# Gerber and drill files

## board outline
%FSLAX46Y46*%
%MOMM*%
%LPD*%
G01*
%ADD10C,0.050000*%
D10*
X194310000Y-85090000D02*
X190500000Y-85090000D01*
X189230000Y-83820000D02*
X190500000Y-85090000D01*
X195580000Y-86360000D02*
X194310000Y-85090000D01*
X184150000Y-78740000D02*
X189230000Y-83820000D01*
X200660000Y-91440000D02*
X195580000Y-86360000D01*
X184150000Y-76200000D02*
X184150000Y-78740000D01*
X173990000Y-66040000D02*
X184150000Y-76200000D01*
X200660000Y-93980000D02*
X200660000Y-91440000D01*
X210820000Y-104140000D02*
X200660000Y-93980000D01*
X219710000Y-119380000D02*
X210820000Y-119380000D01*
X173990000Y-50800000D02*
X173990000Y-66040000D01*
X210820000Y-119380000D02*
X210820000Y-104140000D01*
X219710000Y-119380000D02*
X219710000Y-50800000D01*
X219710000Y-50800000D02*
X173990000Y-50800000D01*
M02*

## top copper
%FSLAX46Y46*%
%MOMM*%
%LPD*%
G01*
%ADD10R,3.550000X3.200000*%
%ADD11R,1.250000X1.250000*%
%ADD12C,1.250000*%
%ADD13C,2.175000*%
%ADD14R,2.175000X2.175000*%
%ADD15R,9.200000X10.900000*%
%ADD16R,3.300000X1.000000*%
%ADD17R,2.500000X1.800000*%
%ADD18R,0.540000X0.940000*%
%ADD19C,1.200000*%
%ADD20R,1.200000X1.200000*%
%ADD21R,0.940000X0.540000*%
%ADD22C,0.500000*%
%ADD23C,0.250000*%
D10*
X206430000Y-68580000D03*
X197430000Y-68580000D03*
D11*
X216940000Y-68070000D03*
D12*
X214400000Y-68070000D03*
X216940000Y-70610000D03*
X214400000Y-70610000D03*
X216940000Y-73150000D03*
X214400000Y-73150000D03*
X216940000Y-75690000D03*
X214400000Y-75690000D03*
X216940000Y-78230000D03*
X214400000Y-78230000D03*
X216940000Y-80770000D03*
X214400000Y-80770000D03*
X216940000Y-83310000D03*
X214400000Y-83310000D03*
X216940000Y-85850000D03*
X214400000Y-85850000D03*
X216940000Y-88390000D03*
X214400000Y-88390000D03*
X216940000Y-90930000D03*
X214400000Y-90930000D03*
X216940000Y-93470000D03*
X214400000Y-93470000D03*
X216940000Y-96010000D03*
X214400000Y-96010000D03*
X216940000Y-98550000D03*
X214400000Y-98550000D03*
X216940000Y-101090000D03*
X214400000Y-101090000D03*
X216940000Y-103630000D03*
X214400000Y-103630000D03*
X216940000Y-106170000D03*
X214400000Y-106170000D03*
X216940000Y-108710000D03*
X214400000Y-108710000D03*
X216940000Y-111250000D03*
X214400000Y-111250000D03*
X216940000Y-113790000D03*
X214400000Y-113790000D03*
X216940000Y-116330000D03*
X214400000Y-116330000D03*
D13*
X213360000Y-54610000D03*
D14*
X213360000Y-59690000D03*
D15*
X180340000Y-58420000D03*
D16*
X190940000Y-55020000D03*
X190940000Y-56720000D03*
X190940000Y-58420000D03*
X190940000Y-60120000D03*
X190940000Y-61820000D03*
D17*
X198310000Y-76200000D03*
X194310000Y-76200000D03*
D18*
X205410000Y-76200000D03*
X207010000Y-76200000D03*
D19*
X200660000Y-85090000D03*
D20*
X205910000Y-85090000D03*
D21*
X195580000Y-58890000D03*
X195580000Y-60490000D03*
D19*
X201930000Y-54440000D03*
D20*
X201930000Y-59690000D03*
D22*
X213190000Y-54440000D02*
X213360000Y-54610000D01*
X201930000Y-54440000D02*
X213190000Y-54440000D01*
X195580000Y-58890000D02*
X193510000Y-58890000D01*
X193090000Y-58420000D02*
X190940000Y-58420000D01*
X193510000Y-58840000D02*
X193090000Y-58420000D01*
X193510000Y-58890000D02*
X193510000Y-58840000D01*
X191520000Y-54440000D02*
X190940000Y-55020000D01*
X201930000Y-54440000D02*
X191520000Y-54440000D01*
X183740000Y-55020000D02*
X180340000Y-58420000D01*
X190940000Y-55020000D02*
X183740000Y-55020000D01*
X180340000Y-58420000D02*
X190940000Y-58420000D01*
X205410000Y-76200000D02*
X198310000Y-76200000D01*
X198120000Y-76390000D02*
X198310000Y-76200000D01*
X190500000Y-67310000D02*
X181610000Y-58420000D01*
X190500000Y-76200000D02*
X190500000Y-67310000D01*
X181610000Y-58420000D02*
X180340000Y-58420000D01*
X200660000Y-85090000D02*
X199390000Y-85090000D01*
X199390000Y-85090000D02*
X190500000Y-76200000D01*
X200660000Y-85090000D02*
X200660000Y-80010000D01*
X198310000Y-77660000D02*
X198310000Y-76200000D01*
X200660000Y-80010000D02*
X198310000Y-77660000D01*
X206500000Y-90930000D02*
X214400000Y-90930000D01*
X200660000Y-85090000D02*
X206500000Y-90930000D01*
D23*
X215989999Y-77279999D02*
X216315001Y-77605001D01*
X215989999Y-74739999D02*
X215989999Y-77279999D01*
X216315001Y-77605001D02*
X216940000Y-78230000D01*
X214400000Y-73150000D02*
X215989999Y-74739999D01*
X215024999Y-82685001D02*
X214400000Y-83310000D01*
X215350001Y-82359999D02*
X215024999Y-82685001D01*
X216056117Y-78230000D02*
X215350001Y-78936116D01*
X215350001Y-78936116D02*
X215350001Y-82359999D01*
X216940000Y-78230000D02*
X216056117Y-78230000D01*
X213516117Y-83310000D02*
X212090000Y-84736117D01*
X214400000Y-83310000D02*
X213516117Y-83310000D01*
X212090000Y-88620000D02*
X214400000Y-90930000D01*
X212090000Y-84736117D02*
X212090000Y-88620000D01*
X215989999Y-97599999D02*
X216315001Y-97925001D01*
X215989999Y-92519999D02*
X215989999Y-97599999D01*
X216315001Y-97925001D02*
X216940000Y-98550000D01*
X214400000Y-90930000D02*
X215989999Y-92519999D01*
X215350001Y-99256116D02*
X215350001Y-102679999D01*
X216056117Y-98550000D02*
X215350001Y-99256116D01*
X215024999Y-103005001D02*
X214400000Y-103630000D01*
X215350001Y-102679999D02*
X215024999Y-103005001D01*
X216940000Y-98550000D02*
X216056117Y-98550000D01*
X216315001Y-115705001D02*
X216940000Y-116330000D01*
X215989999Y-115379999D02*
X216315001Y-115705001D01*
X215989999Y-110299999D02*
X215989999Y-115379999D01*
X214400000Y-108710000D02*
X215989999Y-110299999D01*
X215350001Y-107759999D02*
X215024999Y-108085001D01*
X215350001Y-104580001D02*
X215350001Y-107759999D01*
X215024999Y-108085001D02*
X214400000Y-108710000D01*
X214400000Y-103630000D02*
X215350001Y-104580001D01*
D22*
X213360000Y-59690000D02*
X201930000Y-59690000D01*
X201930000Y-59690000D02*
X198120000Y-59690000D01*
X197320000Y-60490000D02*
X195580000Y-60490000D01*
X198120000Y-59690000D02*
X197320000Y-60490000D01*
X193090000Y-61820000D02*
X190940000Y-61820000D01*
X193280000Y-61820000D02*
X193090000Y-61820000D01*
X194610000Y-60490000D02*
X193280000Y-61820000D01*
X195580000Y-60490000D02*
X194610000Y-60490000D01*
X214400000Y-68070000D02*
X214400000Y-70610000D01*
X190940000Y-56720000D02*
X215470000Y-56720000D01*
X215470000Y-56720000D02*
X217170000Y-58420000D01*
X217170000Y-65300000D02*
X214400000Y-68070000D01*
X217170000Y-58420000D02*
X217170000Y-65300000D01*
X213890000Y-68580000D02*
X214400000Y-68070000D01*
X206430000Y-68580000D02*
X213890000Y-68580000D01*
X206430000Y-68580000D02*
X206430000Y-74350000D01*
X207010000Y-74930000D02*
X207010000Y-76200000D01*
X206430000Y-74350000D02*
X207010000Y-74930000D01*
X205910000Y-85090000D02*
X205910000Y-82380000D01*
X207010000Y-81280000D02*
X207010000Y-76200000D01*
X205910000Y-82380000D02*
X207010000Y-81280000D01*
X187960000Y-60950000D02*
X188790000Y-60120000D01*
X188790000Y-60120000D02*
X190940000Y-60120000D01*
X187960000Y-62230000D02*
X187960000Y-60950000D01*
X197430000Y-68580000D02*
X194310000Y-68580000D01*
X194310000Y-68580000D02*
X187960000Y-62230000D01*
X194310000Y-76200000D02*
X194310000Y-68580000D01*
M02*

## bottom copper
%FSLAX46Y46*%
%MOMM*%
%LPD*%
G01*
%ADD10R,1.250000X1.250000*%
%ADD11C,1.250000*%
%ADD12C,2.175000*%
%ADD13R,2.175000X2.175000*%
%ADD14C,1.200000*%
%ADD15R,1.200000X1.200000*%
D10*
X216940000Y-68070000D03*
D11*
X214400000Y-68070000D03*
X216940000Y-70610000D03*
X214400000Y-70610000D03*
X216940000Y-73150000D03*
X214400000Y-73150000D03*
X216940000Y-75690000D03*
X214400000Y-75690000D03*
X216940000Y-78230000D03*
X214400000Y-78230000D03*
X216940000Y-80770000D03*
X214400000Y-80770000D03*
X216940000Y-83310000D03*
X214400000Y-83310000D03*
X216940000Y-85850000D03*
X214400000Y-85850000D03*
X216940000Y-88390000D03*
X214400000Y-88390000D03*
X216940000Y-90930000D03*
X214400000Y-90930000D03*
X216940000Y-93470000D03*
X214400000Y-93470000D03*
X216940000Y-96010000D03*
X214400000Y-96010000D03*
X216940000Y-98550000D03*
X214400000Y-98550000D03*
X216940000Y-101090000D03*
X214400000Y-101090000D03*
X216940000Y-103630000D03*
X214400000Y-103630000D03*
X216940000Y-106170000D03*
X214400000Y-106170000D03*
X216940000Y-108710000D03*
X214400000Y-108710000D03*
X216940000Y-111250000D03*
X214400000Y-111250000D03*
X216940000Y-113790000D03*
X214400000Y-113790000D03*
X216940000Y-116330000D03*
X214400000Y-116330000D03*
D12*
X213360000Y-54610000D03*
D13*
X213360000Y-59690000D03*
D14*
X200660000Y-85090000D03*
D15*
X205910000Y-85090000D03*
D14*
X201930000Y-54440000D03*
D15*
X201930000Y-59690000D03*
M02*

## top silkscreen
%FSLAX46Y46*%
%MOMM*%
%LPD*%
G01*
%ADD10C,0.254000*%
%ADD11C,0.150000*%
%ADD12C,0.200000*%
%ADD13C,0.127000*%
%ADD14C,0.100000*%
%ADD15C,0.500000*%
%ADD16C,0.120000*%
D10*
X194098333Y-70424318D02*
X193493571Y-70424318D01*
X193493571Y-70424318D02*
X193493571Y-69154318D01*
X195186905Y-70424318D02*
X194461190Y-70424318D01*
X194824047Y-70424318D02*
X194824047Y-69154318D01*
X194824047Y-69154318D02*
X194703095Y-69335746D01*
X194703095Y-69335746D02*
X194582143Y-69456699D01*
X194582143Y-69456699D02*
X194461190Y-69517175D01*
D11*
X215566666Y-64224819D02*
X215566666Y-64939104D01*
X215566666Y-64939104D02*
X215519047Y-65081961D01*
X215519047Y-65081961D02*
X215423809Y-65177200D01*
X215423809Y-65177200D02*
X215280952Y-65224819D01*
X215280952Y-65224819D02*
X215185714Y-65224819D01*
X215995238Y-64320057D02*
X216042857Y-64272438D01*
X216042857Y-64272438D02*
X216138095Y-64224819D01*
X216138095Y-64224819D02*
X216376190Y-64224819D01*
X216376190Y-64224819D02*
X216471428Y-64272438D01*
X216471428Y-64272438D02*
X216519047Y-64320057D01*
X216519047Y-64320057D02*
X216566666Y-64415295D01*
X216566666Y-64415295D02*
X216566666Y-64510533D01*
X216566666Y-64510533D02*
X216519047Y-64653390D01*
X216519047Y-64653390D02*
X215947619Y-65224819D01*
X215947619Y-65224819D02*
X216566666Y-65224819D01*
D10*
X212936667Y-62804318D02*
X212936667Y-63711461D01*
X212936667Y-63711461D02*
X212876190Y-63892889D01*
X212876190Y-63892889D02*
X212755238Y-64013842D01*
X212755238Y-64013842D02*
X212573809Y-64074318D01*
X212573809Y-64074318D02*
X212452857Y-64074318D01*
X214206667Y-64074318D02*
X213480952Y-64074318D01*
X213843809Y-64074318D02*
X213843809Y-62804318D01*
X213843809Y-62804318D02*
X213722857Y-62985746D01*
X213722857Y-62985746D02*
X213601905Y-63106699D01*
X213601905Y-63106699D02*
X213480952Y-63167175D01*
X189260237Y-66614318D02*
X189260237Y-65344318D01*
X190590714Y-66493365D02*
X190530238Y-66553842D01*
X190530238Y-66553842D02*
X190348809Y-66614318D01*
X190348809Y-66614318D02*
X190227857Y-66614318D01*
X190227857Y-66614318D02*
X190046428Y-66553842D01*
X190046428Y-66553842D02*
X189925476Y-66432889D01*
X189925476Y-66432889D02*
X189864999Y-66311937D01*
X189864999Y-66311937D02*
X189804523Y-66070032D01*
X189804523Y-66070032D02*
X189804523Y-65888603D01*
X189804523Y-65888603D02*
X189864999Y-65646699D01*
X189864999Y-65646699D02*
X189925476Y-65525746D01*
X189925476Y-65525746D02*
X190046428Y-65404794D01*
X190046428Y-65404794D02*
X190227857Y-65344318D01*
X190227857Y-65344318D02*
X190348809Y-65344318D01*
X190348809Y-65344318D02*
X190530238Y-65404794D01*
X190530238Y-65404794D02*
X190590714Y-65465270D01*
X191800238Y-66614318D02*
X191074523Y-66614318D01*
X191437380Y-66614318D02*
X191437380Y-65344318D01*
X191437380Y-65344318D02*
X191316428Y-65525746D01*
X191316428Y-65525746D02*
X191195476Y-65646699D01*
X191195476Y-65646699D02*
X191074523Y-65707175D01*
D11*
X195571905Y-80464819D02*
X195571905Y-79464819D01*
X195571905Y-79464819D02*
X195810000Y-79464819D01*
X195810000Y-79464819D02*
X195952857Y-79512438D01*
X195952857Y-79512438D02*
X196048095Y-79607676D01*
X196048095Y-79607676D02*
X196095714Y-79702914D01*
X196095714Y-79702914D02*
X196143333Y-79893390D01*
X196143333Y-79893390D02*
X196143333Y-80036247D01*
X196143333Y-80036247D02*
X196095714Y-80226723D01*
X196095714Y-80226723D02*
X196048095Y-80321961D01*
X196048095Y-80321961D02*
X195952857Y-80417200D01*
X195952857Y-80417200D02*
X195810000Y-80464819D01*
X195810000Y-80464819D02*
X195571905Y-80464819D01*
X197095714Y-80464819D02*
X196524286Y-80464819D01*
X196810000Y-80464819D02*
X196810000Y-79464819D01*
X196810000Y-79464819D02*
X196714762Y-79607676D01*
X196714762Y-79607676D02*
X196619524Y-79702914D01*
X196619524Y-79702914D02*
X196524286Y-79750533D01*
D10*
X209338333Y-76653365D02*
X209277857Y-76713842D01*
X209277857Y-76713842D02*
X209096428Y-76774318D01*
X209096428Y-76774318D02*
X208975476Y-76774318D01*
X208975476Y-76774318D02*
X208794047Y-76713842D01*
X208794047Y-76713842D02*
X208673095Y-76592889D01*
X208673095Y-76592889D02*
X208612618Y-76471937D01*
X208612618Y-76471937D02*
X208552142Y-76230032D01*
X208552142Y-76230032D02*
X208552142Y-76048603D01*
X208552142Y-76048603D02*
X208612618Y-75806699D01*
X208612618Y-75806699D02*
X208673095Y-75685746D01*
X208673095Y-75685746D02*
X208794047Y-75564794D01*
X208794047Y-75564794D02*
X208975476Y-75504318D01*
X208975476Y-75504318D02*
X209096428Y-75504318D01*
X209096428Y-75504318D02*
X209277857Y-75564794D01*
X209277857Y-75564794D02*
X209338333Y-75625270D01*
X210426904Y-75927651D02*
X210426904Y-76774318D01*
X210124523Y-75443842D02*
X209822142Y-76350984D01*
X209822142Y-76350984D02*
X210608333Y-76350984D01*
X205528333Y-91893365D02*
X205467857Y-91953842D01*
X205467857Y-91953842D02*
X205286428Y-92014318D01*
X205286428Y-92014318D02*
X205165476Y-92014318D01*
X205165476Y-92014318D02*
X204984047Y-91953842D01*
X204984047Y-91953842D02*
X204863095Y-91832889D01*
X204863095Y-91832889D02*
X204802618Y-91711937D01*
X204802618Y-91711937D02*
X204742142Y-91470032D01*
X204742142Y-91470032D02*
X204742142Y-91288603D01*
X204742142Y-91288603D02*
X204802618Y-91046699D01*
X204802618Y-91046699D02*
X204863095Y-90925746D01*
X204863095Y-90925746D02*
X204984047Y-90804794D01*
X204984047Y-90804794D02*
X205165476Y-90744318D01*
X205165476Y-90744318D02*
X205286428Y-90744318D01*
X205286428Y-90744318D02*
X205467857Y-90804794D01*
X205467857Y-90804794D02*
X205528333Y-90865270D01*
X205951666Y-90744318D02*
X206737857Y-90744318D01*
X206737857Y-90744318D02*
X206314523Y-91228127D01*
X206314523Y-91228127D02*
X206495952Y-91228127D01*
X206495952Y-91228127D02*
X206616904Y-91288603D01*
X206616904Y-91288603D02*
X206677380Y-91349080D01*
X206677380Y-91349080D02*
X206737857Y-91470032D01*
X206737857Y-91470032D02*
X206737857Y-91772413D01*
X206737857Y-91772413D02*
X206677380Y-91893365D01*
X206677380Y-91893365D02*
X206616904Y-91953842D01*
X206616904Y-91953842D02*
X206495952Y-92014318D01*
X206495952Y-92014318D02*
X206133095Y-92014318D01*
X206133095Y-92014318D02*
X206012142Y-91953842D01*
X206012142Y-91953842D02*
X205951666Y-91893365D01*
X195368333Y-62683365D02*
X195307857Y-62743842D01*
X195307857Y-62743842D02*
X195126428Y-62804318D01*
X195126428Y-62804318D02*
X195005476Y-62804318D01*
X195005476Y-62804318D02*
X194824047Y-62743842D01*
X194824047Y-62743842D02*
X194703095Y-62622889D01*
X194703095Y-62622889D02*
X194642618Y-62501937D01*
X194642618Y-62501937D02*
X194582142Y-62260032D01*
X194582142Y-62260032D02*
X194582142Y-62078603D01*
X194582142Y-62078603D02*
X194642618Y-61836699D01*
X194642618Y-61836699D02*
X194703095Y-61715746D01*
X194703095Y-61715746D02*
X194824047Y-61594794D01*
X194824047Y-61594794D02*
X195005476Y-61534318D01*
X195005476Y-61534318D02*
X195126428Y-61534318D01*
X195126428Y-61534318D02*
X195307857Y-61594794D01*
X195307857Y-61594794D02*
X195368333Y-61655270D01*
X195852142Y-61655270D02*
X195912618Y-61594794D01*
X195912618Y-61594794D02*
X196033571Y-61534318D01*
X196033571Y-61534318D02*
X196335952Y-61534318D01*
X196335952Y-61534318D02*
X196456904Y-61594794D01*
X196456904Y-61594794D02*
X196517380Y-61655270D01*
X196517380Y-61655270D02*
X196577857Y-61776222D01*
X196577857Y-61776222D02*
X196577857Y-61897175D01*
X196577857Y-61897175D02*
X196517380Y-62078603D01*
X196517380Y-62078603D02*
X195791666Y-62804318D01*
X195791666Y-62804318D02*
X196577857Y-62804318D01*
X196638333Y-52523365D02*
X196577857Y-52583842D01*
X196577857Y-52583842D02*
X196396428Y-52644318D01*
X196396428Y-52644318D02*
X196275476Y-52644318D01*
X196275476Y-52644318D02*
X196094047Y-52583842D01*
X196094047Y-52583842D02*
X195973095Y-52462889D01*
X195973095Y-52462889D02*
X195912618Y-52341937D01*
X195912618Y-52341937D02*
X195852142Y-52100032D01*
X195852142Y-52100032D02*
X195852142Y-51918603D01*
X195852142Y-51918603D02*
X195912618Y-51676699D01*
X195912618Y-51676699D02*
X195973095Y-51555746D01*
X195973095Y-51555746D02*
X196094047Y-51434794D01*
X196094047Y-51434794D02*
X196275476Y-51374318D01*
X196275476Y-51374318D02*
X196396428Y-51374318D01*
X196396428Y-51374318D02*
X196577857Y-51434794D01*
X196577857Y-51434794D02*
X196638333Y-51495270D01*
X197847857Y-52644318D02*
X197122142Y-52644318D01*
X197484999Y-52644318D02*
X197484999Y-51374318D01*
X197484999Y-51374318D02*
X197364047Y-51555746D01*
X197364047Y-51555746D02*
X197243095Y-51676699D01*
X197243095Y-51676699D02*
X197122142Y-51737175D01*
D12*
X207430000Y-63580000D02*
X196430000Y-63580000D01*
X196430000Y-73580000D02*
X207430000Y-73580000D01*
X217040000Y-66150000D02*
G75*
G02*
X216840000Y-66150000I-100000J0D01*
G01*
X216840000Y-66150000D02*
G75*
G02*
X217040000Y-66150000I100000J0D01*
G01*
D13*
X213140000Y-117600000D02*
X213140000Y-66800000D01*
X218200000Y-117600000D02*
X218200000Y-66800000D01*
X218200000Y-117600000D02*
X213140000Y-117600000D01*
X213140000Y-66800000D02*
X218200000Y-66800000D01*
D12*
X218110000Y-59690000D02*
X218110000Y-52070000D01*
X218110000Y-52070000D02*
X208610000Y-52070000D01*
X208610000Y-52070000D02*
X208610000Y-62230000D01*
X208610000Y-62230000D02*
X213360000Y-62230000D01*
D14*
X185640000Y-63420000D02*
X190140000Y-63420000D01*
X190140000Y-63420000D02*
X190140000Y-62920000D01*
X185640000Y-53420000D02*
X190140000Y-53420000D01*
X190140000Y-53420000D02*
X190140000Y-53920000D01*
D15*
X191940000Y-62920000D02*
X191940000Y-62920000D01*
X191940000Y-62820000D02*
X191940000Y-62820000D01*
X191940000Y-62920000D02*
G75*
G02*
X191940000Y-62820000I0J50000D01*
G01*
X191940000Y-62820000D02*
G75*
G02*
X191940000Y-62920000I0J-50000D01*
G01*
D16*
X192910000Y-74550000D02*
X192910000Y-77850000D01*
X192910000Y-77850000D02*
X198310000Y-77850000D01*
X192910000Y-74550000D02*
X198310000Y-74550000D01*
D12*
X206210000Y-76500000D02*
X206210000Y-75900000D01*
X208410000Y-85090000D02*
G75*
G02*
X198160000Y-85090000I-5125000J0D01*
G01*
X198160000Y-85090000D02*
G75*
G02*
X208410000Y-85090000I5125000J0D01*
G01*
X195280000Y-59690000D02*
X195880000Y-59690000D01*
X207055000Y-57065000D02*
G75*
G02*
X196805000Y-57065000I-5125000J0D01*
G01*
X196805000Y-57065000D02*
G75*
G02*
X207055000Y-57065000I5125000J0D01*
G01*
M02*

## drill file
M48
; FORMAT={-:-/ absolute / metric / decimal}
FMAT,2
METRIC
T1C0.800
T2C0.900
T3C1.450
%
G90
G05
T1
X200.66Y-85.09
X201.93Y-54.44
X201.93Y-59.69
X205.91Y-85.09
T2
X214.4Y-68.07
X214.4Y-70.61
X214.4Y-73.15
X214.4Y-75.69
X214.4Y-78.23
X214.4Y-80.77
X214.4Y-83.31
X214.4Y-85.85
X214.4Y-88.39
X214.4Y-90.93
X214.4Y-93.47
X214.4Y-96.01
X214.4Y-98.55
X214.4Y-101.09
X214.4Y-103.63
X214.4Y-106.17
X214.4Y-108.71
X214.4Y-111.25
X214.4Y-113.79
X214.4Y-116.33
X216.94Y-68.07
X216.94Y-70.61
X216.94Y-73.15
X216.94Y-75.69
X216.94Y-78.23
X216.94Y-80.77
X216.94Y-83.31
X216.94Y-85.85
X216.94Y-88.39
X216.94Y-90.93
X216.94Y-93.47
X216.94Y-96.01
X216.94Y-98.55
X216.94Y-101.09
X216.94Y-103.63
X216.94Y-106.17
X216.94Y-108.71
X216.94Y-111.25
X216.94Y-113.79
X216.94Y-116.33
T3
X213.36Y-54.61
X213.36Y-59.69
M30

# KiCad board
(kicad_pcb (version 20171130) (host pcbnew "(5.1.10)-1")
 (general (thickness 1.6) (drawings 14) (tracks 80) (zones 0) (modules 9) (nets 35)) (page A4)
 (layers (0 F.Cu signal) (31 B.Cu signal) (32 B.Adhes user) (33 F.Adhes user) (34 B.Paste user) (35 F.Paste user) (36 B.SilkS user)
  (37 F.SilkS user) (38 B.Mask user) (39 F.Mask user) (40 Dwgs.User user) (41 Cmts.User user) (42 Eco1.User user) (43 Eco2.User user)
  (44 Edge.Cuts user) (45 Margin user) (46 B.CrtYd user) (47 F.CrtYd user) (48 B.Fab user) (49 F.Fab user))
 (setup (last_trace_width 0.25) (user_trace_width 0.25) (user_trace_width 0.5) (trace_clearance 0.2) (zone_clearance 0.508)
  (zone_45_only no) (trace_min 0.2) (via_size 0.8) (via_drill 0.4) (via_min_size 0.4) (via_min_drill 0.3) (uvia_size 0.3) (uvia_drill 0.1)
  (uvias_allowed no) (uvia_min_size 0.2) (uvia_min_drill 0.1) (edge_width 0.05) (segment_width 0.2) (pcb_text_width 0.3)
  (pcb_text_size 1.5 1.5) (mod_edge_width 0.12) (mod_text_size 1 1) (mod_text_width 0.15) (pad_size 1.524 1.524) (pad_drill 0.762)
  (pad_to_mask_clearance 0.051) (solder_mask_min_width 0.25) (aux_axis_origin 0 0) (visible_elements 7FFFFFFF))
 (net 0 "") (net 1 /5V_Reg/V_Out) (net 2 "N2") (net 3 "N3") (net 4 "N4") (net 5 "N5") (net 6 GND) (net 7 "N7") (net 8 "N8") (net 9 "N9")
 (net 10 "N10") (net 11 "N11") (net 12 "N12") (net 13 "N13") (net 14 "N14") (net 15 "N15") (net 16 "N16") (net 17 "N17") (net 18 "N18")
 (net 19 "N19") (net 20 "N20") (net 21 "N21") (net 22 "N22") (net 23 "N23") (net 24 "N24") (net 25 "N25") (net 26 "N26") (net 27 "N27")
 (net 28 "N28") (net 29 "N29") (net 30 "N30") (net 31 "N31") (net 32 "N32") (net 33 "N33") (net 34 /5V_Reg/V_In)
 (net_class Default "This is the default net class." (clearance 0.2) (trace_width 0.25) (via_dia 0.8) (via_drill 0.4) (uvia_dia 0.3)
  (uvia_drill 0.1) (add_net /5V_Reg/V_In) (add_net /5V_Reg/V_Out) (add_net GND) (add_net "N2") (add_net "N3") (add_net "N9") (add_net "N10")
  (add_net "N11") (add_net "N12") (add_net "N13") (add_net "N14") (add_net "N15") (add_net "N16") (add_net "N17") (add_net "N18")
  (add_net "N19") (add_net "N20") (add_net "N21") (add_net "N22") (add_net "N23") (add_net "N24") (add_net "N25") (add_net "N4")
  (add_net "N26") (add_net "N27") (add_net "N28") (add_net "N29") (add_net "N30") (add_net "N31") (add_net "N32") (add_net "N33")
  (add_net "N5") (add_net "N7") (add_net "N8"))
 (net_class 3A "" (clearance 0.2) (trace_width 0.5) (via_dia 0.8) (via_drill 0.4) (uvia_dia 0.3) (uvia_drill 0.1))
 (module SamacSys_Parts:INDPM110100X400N (layer F.Cu) (at 201.93 68.58)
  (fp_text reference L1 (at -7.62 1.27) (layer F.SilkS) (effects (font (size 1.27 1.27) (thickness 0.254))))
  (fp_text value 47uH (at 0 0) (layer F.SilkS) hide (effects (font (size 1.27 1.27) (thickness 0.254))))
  (fp_line (start 5.5 -5) (end -5.5 -5) (layer F.SilkS) (width 0.2))
  (fp_line (start -5.5 5) (end 5.5 5) (layer F.SilkS) (width 0.2))
  (pad 2 smd rect (at 4.5 0 90) (size 3.2 3.55) (layers F.Cu F.Paste F.Mask) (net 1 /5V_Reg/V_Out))
  (pad 1 smd rect (at -4.5 0 90) (size 3.2 3.55) (layers F.Cu F.Paste F.Mask) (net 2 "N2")))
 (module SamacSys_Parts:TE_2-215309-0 (layer F.Cu) (at 216.94 68.07 270)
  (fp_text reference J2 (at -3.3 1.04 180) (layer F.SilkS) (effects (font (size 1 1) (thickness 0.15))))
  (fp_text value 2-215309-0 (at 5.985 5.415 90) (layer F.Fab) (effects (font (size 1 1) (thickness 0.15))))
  (fp_circle (center -1.92 0) (end -1.82 0) (layer F.SilkS) (width 0.2))
  (fp_line (start 49.53 3.8) (end -1.27 3.8) (layer F.SilkS) (width 0.127))
  (fp_line (start 49.53 -1.26) (end -1.27 -1.26) (layer F.SilkS) (width 0.127))
  (fp_line (start 49.53 -1.26) (end 49.53 3.8) (layer F.SilkS) (width 0.127))
  (fp_line (start -1.27 3.8) (end -1.27 -1.26) (layer F.SilkS) (width 0.127))
  (pad 1 thru_hole rect (at 0 0 270) (size 1.25 1.25) (drill 0.9) (layers *.Cu *.Mask) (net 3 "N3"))
  (pad 2 thru_hole circle (at 0 2.54 270) (size 1.25 1.25) (drill 0.9) (layers *.Cu *.Mask) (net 1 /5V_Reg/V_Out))
  (pad 3 thru_hole circle (at 2.54 0 270) (size 1.25 1.25) (drill 0.9) (layers *.Cu *.Mask) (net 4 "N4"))
  (pad 4 thru_hole circle (at 2.54 2.54 270) (size 1.25 1.25) (drill 0.9) (layers *.Cu *.Mask) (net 1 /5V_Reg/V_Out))
  (pad 5 thru_hole circle (at 5.08 0 270) (size 1.25 1.25) (drill 0.9) (layers *.Cu *.Mask) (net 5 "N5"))
  (pad 6 thru_hole circle (at 5.08 2.54 270) (size 1.25 1.25) (drill 0.9) (layers *.Cu *.Mask) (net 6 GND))
  (pad 7 thru_hole circle (at 7.62 0 270) (size 1.25 1.25) (drill 0.9) (layers *.Cu *.Mask) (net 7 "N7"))
  (pad 8 thru_hole circle (at 7.62 2.54 270) (size 1.25 1.25) (drill 0.9) (layers *.Cu *.Mask) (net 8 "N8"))
  (pad 9 thru_hole circle (at 10.16 0 270) (size 1.25 1.25) (drill 0.9) (layers *.Cu *.Mask) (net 6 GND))
  (pad 10 thru_hole circle (at 10.16 2.54 270) (size 1.25 1.25) (drill 0.9) (layers *.Cu *.Mask) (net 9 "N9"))
  (pad 11 thru_hole circle (at 12.7 0 270) (size 1.25 1.25) (drill 0.9) (layers *.Cu *.Mask) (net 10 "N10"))
  (pad 12 thru_hole circle (at 12.7 2.54 270) (size 1.25 1.25) (drill 0.9) (layers *.Cu *.Mask) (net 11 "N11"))
  (pad 13 thru_hole circle (at 15.24 0 270) (size 1.25 1.25) (drill 0.9) (layers *.Cu *.Mask) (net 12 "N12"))
  (pad 14 thru_hole circle (at 15.24 2.54 270) (size 1.25 1.25) (drill 0.9) (layers *.Cu *.Mask) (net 6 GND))
  (pad 15 thru_hole circle (at 17.78 0 270) (size 1.25 1.25) (drill 0.9) (layers *.Cu *.Mask) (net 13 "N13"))
  (pad 16 thru_hole circle (at 17.78 2.54 270) (size 1.25 1.25) (drill 0.9) (layers *.Cu *.Mask) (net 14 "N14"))
  (pad 17 thru_hole circle (at 20.32 0 270) (size 1.25 1.25) (drill 0.9) (layers *.Cu *.Mask) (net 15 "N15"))
  (pad 18 thru_hole circle (at 20.32 2.54 270) (size 1.25 1.25) (drill 0.9) (layers *.Cu *.Mask) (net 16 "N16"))
  (pad 19 thru_hole circle (at 22.86 0 270) (size 1.25 1.25) (drill 0.9) (layers *.Cu *.Mask) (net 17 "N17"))
  (pad 20 thru_hole circle (at 22.86 2.54 270) (size 1.25 1.25) (drill 0.9) (layers *.Cu *.Mask) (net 6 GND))
  (pad 21 thru_hole circle (at 25.4 0 270) (size 1.25 1.25) (drill 0.9) (layers *.Cu *.Mask) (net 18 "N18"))
  (pad 22 thru_hole circle (at 25.4 2.54 270) (size 1.25 1.25) (drill 0.9) (layers *.Cu *.Mask) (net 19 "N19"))
  (pad 23 thru_hole circle (at 27.94 0 270) (size 1.25 1.25) (drill 0.9) (layers *.Cu *.Mask) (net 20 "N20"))
  (pad 24 thru_hole circle (at 27.94 2.54 270) (size 1.25 1.25) (drill 0.9) (layers *.Cu *.Mask) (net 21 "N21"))
  (pad 25 thru_hole circle (at 30.48 0 270) (size 1.25 1.25) (drill 0.9) (layers *.Cu *.Mask) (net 6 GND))
  (pad 26 thru_hole circle (at 30.48 2.54 270) (size 1.25 1.25) (drill 0.9) (layers *.Cu *.Mask) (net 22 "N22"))
  (pad 27 thru_hole circle (at 33.02 0 270) (size 1.25 1.25) (drill 0.9) (layers *.Cu *.Mask) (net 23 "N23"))
  (pad 28 thru_hole circle (at 33.02 2.54 270) (size 1.25 1.25) (drill 0.9) (layers *.Cu *.Mask) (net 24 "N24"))
  (pad 29 thru_hole circle (at 35.56 0 270) (size 1.25 1.25) (drill 0.9) (layers *.Cu *.Mask) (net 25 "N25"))
  (pad 30 thru_hole circle (at 35.56 2.54 270) (size 1.25 1.25) (drill 0.9) (layers *.Cu *.Mask) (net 6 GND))
  (pad 31 thru_hole circle (at 38.1 0 270) (size 1.25 1.25) (drill 0.9) (layers *.Cu *.Mask) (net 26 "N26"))
  (pad 32 thru_hole circle (at 38.1 2.54 270) (size 1.25 1.25) (drill 0.9) (layers *.Cu *.Mask) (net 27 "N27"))
  (pad 33 thru_hole circle (at 40.64 0 270) (size 1.25 1.25) (drill 0.9) (layers *.Cu *.Mask) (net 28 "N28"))
  (pad 34 thru_hole circle (at 40.64 2.54 270) (size 1.25 1.25) (drill 0.9) (layers *.Cu *.Mask) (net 6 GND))
  (pad 35 thru_hole circle (at 43.18 0 270) (size 1.25 1.25) (drill 0.9) (layers *.Cu *.Mask) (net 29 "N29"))
  (pad 36 thru_hole circle (at 43.18 2.54 270) (size 1.25 1.25) (drill 0.9) (layers *.Cu *.Mask) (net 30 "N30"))
  (pad 37 thru_hole circle (at 45.72 0 270) (size 1.25 1.25) (drill 0.9) (layers *.Cu *.Mask) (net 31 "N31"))
  (pad 38 thru_hole circle (at 45.72 2.54 270) (size 1.25 1.25) (drill 0.9) (layers *.Cu *.Mask) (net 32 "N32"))
  (pad 39 thru_hole circle (at 48.26 0 270) (size 1.25 1.25) (drill 0.9) (layers *.Cu *.Mask) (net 6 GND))
  (pad 40 thru_hole circle (at 48.26 2.54 270) (size 1.25 1.25) (drill 0.9) (layers *.Cu *.Mask) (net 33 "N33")))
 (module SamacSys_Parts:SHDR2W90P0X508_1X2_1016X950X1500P (layer F.Cu) (at 213.36 59.69 90)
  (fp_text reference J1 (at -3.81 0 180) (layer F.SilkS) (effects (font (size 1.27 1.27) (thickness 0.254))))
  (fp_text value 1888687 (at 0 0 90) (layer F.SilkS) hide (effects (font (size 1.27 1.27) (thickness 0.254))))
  (fp_line (start 0 4.75) (end 7.62 4.75) (layer F.SilkS) (width 0.2))
  (fp_line (start 7.62 4.75) (end 7.62 -4.75) (layer F.SilkS) (width 0.2))
  (fp_line (start 7.62 -4.75) (end -2.54 -4.75) (layer F.SilkS) (width 0.2))
  (fp_line (start -2.54 -4.75) (end -2.54 0) (layer F.SilkS) (width 0.2))
  (pad 2 thru_hole circle (at 5.08 0 90) (size 2.175 2.175) (drill 1.45) (layers *.Cu *.Mask) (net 6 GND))
  (pad 1 thru_hole rect (at 0 0 90) (size 2.175 2.175) (drill 1.45) (layers *.Cu *.Mask) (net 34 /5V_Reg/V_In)))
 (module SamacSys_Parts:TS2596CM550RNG (layer F.Cu) (at 185.64 58.42 90)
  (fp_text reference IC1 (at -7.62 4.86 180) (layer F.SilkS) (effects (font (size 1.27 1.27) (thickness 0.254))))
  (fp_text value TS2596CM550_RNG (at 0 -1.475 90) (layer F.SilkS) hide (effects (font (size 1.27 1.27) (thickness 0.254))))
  (fp_line (start -5 0) (end -5 4.5) (layer F.SilkS) (width 0.1))
  (fp_line (start -5 4.5) (end -4.5 4.5) (layer F.SilkS) (width 0.1))
  (fp_line (start 5 0) (end 5 4.5) (layer F.SilkS) (width 0.1))
  (fp_line (start 5 4.5) (end 4.5 4.5) (layer F.SilkS) (width 0.1))
  (fp_line (start -4.5 6.3) (end -4.5 6.3) (layer F.SilkS) (width 0.5))
  (fp_line (start -4.4 6.3) (end -4.4 6.3) (layer F.SilkS) (width 0.5))
  (fp_arc (start -4.45 6.3) (end -4.4 6.3) (angle -180) (layer F.SilkS) (width 0.5))
  (fp_arc (start -4.45 6.3) (end -4.5 6.3) (angle -180) (layer F.SilkS) (width 0.5))
  (pad 6 smd rect (at 0 -5.3 180) (size 9.2 10.9) (layers F.Cu F.Paste F.Mask) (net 6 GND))
  (pad 5 smd rect (at 3.4 5.3 90) (size 1 3.3) (layers F.Cu F.Paste F.Mask) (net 6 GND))
  (pad 4 smd rect (at 1.7 5.3 90) (size 1 3.3) (layers F.Cu F.Paste F.Mask) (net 1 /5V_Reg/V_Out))
  (pad 3 smd rect (at 0 5.3 90) (size 1 3.3) (layers F.Cu F.Paste F.Mask) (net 6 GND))
  (pad 2 smd rect (at -1.7 5.3 90) (size 1 3.3) (layers F.Cu F.Paste F.Mask) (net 2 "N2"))
  (pad 1 smd rect (at -3.4 5.3 90) (size 1 3.3) (layers F.Cu F.Paste F.Mask) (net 34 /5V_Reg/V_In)))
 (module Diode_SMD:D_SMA (layer F.Cu) (at 196.31 76.2)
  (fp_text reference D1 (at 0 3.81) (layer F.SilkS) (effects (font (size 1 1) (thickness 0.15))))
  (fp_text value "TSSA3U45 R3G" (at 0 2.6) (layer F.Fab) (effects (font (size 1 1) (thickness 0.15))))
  (fp_line (start -3.4 -1.65) (end -3.4 1.65) (layer F.SilkS) (width 0.12))
  (fp_line (start -3.4 1.65) (end 2 1.65) (layer F.SilkS) (width 0.12))
  (fp_line (start -3.4 -1.65) (end 2 -1.65) (layer F.SilkS) (width 0.12))
  (pad 2 smd rect (at 2 0) (size 2.5 1.8) (layers F.Cu F.Paste F.Mask) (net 6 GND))
  (pad 1 smd rect (at -2 0) (size 2.5 1.8) (layers F.Cu F.Paste F.Mask) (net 2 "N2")))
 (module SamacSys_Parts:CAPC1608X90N (layer F.Cu) (at 206.21 76.2 180)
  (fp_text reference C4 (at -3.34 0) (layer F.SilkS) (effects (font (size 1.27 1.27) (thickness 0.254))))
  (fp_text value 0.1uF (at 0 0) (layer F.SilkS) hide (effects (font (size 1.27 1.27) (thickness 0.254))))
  (fp_line (start 0 -0.3) (end 0 0.3) (layer F.SilkS) (width 0.2))
  (pad 2 smd rect (at 0.8 0 180) (size 0.54 0.94) (layers F.Cu F.Paste F.Mask) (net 6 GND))
  (pad 1 smd rect (at -0.8 0 180) (size 0.54 0.94) (layers F.Cu F.Paste F.Mask) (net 1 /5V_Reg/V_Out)))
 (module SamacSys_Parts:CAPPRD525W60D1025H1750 (layer F.Cu) (at 205.91 85.09 180)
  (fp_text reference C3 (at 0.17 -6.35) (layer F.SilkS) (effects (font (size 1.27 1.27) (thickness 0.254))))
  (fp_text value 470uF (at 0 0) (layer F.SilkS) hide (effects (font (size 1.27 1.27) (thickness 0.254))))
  (fp_circle (center 2.625 0) (end 2.625 5.125) (layer F.SilkS) (width 0.2))
  (pad 2 thru_hole circle (at 5.25 0 180) (size 1.2 1.2) (drill 0.8) (layers *.Cu *.Mask) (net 6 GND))
  (pad 1 thru_hole rect (at 0 0 180) (size 1.2 1.2) (drill 0.8) (layers *.Cu *.Mask) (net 1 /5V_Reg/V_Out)))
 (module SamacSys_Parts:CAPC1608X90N (layer F.Cu) (at 195.58 59.69 90)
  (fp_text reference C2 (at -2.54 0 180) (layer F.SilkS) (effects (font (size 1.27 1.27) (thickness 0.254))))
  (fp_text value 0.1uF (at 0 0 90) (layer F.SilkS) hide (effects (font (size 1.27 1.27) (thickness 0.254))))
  (fp_line (start 0 -0.3) (end 0 0.3) (layer F.SilkS) (width 0.2))
  (pad 2 smd rect (at 0.8 0 90) (size 0.54 0.94) (layers F.Cu F.Paste F.Mask) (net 6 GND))
  (pad 1 smd rect (at -0.8 0 90) (size 0.54 0.94) (layers F.Cu F.Paste F.Mask) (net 34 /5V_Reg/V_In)))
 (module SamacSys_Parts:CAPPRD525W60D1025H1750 (layer F.Cu) (at 201.93 59.69 90)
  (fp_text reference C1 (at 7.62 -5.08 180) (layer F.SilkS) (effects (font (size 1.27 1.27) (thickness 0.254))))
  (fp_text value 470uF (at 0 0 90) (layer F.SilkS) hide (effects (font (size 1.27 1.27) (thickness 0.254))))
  (fp_circle (center 2.625 0) (end 2.625 5.125) (layer F.SilkS) (width 0.2))
  (pad 2 thru_hole circle (at 5.25 0 90) (size 1.2 1.2) (drill 0.8) (layers *.Cu *.Mask) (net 6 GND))
  (pad 1 thru_hole rect (at 0 0 90) (size 1.2 1.2) (drill 0.8) (layers *.Cu *.Mask) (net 34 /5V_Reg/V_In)))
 (gr_line (start 194.31 85.09) (end 190.5 85.09) (layer Edge.Cuts) (width 0.05))
 (gr_line (start 189.23 83.82) (end 190.5 85.09) (layer Edge.Cuts) (width 0.05))
 (gr_line (start 195.58 86.36) (end 194.31 85.09) (layer Edge.Cuts) (width 0.05))
 (gr_line (start 184.15 78.74) (end 189.23 83.82) (layer Edge.Cuts) (width 0.05))
 (gr_line (start 200.66 91.44) (end 195.58 86.36) (layer Edge.Cuts) (width 0.05))
 (gr_line (start 184.15 76.2) (end 184.15 78.74) (layer Edge.Cuts) (width 0.05))
 (gr_line (start 173.99 66.04) (end 184.15 76.2) (layer Edge.Cuts) (width 0.05))
 (gr_line (start 200.66 93.98) (end 200.66 91.44) (layer Edge.Cuts) (width 0.05))
 (gr_line (start 210.82 104.14) (end 200.66 93.98) (layer Edge.Cuts) (width 0.05))
 (gr_line (start 219.71 119.38) (end 210.82 119.38) (layer Edge.Cuts) (width 0.05))
 (gr_line (start 173.99 50.8) (end 173.99 66.04) (layer Edge.Cuts) (width 0.05))
 (gr_line (start 210.82 119.38) (end 210.82 104.14) (layer Edge.Cuts) (width 0.05))
 (gr_line (start 219.71 119.38) (end 219.71 50.8) (layer Edge.Cuts) (width 0.05))
 (gr_line (start 219.71 50.8) (end 173.99 50.8) (layer Edge.Cuts) (width 0.05))
 (segment (start 213.19 54.44) (end 213.36 54.61) (width 0.5) (layer F.Cu) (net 6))
 (segment (start 201.93 54.44) (end 213.19 54.44) (width 0.5) (layer F.Cu) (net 6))
 (segment (start 195.58 58.89) (end 193.51 58.89) (width 0.5) (layer F.Cu) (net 6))
 (segment (start 193.09 58.42) (end 190.94 58.42) (width 0.5) (layer F.Cu) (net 6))
 (segment (start 193.51 58.84) (end 193.09 58.42) (width 0.5) (layer F.Cu) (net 6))
 (segment (start 193.51 58.89) (end 193.51 58.84) (width 0.5) (layer F.Cu) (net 6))
 (segment (start 191.52 54.44) (end 190.94 55.02) (width 0.5) (layer F.Cu) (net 6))
 (segment (start 201.93 54.44) (end 191.52 54.44) (width 0.5) (layer F.Cu) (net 6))
 (segment (start 183.74 55.02) (end 180.34 58.42) (width 0.5) (layer F.Cu) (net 6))
 (segment (start 190.94 55.02) (end 183.74 55.02) (width 0.5) (layer F.Cu) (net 6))
 (segment (start 180.34 58.42) (end 190.94 58.42) (width 0.5) (layer F.Cu) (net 6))
 (segment (start 205.41 76.2) (end 198.31 76.2) (width 0.5) (layer F.Cu) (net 6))
 (segment (start 198.12 76.39) (end 198.31 76.2) (width 0.5) (layer F.Cu) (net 6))
 (segment (start 190.5 67.31) (end 181.61 58.42) (width 0.5) (layer F.Cu) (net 6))
 (segment (start 190.5 76.2) (end 190.5 67.31) (width 0.5) (layer F.Cu) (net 6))
 (segment (start 181.61 58.42) (end 180.34 58.42) (width 0.5) (layer F.Cu) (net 6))
 (segment (start 200.66 85.09) (end 199.39 85.09) (width 0.5) (layer F.Cu) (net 6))
 (segment (start 199.39 85.09) (end 190.5 76.2) (width 0.5) (layer F.Cu) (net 6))
 (segment (start 200.66 85.09) (end 200.66 80.01) (width 0.5) (layer F.Cu) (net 6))
 (segment (start 198.31 77.66) (end 198.31 76.2) (width 0.5) (layer F.Cu) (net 6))
 (segment (start 200.66 80.01) (end 198.31 77.66) (width 0.5) (layer F.Cu) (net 6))
 (segment (start 206.5 90.93) (end 214.4 90.93) (width 0.5) (layer F.Cu) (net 6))
 (segment (start 200.66 85.09) (end 206.5 90.93) (width 0.5) (layer F.Cu) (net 6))
 (segment (start 215.989999 77.279999) (end 216.315001 77.605001) (width 0.25) (layer F.Cu) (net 6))
 (segment (start 215.989999 74.739999) (end 215.989999 77.279999) (width 0.25) (layer F.Cu) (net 6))
 (segment (start 216.315001 77.605001) (end 216.94 78.23) (width 0.25) (layer F.Cu) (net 6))
 (segment (start 214.4 73.15) (end 215.989999 74.739999) (width 0.25) (layer F.Cu) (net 6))
 (segment (start 215.024999 82.685001) (end 214.4 83.31) (width 0.25) (layer F.Cu) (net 6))
 (segment (start 215.350001 82.359999) (end 215.024999 82.685001) (width 0.25) (layer F.Cu) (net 6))
 (segment (start 216.056117 78.23) (end 215.350001 78.936116) (width 0.25) (layer F.Cu) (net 6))
 (segment (start 215.350001 78.936116) (end 215.350001 82.359999) (width 0.25) (layer F.Cu) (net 6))
 (segment (start 216.94 78.23) (end 216.056117 78.23) (width 0.25) (layer F.Cu) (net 6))
 (segment (start 213.516117 83.31) (end 212.09 84.736117) (width 0.25) (layer F.Cu) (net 6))
 (segment (start 214.4 83.31) (end 213.516117 83.31) (width 0.25) (layer F.Cu) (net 6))
 (segment (start 212.09 88.62) (end 214.4 90.93) (width 0.25) (layer F.Cu) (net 6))
 (segment (start 212.09 84.736117) (end 212.09 88.62) (width 0.25) (layer F.Cu) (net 6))
 (segment (start 215.989999 97.599999) (end 216.315001 97.925001) (width 0.25) (layer F.Cu) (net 6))
 (segment (start 215.989999 92.519999) (end 215.989999 97.599999) (width 0.25) (layer F.Cu) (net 6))
 (segment (start 216.315001 97.925001) (end 216.94 98.55) (width 0.25) (layer F.Cu) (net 6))
 (segment (start 214.4 90.93) (end 215.989999 92.519999) (width 0.25) (layer F.Cu) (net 6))
 (segment (start 215.350001 99.256116) (end 215.350001 102.679999) (width 0.25) (layer F.Cu) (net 6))
 (segment (start 216.056117 98.55) (end 215.350001 99.256116) (width 0.25) (layer F.Cu) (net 6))
 (segment (start 215.024999 103.005001) (end 214.4 103.63) (width 0.25) (layer F.Cu) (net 6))
 (segment (start 215.350001 102.679999) (end 215.024999 103.005001) (width 0.25) (layer F.Cu) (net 6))
 (segment (start 216.94 98.55) (end 216.056117 98.55) (width 0.25) (layer F.Cu) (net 6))
 (segment (start 216.315001 115.705001) (end 216.94 116.33) (width 0.25) (layer F.Cu) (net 6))
 (segment (start 215.989999 115.379999) (end 216.315001 115.705001) (width 0.25) (layer F.Cu) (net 6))
 (segment (start 215.989999 110.299999) (end 215.989999 115.379999) (width 0.25) (layer F.Cu) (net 6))
 (segment (start 214.4 108.71) (end 215.989999 110.299999) (width 0.25) (layer F.Cu) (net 6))
 (segment (start 215.350001 107.759999) (end 215.024999 108.085001) (width 0.25) (layer F.Cu) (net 6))
 (segment (start 215.350001 104.580001) (end 215.350001 107.759999) (width 0.25) (layer F.Cu) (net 6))
 (segment (start 215.024999 108.085001) (end 214.4 108.71) (width 0.25) (layer F.Cu) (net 6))
 (segment (start 214.4 103.63) (end 215.350001 104.580001) (width 0.25) (layer F.Cu) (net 6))
 (segment (start 213.36 59.69) (end 201.93 59.69) (width 0.5) (layer F.Cu) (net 34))
 (segment (start 201.93 59.69) (end 198.12 59.69) (width 0.5) (layer F.Cu) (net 34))
 (segment (start 197.32 60.49) (end 195.58 60.49) (width 0.5) (layer F.Cu) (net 34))
 (segment (start 198.12 59.69) (end 197.32 60.49) (width 0.5) (layer F.Cu) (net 34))
 (segment (start 193.09 61.82) (end 190.94 61.82) (width 0.5) (layer F.Cu) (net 34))
 (segment (start 193.28 61.82) (end 193.09 61.82) (width 0.5) (layer F.Cu) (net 34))
 (segment (start 194.61 60.49) (end 193.28 61.82) (width 0.5) (layer F.Cu) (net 34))
 (segment (start 195.58 60.49) (end 194.61 60.49) (width 0.5) (layer F.Cu) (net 34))
 (segment (start 214.4 68.07) (end 214.4 70.61) (width 0.5) (layer F.Cu) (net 1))
 (segment (start 190.94 56.72) (end 215.47 56.72) (width 0.5) (layer F.Cu) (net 1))
 (segment (start 215.47 56.72) (end 217.17 58.42) (width 0.5) (layer F.Cu) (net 1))
 (segment (start 217.17 65.3) (end 214.4 68.07) (width 0.5) (layer F.Cu) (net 1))
 (segment (start 217.17 58.42) (end 217.17 65.3) (width 0.5) (layer F.Cu) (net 1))
 (segment (start 213.89 68.58) (end 214.4 68.07) (width 0.5) (layer F.Cu) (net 1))
 (segment (start 206.43 68.58) (end 213.89 68.58) (width 0.5) (layer F.Cu) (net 1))
 (segment (start 206.43 68.58) (end 206.43 74.35) (width 0.5) (layer F.Cu) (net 1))
 (segment (start 207.01 74.93) (end 207.01 76.2) (width 0.5) (layer F.Cu) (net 1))
 (segment (start 206.43 74.35) (end 207.01 74.93) (width 0.5) (layer F.Cu) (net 1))
 (segment (start 205.91 85.09) (end 205.91 82.38) (width 0.5) (layer F.Cu) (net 1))
 (segment (start 207.01 81.28) (end 207.01 76.2) (width 0.5) (layer F.Cu) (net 1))
 (segment (start 205.91 82.38) (end 207.01 81.28) (width 0.5) (layer F.Cu) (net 1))
 (segment (start 187.96 60.95) (end 188.79 60.12) (width 0.5) (layer F.Cu) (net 2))
 (segment (start 188.79 60.12) (end 190.94 60.12) (width 0.5) (layer F.Cu) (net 2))
 (segment (start 187.96 62.23) (end 187.96 60.95) (width 0.5) (layer F.Cu) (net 2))
 (segment (start 197.43 68.58) (end 194.31 68.58) (width 0.5) (layer F.Cu) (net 2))
 (segment (start 194.31 68.58) (end 187.96 62.23) (width 0.5) (layer F.Cu) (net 2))
 (segment (start 194.31 76.2) (end 194.31 68.58) (width 0.5) (layer F.Cu) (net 2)))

